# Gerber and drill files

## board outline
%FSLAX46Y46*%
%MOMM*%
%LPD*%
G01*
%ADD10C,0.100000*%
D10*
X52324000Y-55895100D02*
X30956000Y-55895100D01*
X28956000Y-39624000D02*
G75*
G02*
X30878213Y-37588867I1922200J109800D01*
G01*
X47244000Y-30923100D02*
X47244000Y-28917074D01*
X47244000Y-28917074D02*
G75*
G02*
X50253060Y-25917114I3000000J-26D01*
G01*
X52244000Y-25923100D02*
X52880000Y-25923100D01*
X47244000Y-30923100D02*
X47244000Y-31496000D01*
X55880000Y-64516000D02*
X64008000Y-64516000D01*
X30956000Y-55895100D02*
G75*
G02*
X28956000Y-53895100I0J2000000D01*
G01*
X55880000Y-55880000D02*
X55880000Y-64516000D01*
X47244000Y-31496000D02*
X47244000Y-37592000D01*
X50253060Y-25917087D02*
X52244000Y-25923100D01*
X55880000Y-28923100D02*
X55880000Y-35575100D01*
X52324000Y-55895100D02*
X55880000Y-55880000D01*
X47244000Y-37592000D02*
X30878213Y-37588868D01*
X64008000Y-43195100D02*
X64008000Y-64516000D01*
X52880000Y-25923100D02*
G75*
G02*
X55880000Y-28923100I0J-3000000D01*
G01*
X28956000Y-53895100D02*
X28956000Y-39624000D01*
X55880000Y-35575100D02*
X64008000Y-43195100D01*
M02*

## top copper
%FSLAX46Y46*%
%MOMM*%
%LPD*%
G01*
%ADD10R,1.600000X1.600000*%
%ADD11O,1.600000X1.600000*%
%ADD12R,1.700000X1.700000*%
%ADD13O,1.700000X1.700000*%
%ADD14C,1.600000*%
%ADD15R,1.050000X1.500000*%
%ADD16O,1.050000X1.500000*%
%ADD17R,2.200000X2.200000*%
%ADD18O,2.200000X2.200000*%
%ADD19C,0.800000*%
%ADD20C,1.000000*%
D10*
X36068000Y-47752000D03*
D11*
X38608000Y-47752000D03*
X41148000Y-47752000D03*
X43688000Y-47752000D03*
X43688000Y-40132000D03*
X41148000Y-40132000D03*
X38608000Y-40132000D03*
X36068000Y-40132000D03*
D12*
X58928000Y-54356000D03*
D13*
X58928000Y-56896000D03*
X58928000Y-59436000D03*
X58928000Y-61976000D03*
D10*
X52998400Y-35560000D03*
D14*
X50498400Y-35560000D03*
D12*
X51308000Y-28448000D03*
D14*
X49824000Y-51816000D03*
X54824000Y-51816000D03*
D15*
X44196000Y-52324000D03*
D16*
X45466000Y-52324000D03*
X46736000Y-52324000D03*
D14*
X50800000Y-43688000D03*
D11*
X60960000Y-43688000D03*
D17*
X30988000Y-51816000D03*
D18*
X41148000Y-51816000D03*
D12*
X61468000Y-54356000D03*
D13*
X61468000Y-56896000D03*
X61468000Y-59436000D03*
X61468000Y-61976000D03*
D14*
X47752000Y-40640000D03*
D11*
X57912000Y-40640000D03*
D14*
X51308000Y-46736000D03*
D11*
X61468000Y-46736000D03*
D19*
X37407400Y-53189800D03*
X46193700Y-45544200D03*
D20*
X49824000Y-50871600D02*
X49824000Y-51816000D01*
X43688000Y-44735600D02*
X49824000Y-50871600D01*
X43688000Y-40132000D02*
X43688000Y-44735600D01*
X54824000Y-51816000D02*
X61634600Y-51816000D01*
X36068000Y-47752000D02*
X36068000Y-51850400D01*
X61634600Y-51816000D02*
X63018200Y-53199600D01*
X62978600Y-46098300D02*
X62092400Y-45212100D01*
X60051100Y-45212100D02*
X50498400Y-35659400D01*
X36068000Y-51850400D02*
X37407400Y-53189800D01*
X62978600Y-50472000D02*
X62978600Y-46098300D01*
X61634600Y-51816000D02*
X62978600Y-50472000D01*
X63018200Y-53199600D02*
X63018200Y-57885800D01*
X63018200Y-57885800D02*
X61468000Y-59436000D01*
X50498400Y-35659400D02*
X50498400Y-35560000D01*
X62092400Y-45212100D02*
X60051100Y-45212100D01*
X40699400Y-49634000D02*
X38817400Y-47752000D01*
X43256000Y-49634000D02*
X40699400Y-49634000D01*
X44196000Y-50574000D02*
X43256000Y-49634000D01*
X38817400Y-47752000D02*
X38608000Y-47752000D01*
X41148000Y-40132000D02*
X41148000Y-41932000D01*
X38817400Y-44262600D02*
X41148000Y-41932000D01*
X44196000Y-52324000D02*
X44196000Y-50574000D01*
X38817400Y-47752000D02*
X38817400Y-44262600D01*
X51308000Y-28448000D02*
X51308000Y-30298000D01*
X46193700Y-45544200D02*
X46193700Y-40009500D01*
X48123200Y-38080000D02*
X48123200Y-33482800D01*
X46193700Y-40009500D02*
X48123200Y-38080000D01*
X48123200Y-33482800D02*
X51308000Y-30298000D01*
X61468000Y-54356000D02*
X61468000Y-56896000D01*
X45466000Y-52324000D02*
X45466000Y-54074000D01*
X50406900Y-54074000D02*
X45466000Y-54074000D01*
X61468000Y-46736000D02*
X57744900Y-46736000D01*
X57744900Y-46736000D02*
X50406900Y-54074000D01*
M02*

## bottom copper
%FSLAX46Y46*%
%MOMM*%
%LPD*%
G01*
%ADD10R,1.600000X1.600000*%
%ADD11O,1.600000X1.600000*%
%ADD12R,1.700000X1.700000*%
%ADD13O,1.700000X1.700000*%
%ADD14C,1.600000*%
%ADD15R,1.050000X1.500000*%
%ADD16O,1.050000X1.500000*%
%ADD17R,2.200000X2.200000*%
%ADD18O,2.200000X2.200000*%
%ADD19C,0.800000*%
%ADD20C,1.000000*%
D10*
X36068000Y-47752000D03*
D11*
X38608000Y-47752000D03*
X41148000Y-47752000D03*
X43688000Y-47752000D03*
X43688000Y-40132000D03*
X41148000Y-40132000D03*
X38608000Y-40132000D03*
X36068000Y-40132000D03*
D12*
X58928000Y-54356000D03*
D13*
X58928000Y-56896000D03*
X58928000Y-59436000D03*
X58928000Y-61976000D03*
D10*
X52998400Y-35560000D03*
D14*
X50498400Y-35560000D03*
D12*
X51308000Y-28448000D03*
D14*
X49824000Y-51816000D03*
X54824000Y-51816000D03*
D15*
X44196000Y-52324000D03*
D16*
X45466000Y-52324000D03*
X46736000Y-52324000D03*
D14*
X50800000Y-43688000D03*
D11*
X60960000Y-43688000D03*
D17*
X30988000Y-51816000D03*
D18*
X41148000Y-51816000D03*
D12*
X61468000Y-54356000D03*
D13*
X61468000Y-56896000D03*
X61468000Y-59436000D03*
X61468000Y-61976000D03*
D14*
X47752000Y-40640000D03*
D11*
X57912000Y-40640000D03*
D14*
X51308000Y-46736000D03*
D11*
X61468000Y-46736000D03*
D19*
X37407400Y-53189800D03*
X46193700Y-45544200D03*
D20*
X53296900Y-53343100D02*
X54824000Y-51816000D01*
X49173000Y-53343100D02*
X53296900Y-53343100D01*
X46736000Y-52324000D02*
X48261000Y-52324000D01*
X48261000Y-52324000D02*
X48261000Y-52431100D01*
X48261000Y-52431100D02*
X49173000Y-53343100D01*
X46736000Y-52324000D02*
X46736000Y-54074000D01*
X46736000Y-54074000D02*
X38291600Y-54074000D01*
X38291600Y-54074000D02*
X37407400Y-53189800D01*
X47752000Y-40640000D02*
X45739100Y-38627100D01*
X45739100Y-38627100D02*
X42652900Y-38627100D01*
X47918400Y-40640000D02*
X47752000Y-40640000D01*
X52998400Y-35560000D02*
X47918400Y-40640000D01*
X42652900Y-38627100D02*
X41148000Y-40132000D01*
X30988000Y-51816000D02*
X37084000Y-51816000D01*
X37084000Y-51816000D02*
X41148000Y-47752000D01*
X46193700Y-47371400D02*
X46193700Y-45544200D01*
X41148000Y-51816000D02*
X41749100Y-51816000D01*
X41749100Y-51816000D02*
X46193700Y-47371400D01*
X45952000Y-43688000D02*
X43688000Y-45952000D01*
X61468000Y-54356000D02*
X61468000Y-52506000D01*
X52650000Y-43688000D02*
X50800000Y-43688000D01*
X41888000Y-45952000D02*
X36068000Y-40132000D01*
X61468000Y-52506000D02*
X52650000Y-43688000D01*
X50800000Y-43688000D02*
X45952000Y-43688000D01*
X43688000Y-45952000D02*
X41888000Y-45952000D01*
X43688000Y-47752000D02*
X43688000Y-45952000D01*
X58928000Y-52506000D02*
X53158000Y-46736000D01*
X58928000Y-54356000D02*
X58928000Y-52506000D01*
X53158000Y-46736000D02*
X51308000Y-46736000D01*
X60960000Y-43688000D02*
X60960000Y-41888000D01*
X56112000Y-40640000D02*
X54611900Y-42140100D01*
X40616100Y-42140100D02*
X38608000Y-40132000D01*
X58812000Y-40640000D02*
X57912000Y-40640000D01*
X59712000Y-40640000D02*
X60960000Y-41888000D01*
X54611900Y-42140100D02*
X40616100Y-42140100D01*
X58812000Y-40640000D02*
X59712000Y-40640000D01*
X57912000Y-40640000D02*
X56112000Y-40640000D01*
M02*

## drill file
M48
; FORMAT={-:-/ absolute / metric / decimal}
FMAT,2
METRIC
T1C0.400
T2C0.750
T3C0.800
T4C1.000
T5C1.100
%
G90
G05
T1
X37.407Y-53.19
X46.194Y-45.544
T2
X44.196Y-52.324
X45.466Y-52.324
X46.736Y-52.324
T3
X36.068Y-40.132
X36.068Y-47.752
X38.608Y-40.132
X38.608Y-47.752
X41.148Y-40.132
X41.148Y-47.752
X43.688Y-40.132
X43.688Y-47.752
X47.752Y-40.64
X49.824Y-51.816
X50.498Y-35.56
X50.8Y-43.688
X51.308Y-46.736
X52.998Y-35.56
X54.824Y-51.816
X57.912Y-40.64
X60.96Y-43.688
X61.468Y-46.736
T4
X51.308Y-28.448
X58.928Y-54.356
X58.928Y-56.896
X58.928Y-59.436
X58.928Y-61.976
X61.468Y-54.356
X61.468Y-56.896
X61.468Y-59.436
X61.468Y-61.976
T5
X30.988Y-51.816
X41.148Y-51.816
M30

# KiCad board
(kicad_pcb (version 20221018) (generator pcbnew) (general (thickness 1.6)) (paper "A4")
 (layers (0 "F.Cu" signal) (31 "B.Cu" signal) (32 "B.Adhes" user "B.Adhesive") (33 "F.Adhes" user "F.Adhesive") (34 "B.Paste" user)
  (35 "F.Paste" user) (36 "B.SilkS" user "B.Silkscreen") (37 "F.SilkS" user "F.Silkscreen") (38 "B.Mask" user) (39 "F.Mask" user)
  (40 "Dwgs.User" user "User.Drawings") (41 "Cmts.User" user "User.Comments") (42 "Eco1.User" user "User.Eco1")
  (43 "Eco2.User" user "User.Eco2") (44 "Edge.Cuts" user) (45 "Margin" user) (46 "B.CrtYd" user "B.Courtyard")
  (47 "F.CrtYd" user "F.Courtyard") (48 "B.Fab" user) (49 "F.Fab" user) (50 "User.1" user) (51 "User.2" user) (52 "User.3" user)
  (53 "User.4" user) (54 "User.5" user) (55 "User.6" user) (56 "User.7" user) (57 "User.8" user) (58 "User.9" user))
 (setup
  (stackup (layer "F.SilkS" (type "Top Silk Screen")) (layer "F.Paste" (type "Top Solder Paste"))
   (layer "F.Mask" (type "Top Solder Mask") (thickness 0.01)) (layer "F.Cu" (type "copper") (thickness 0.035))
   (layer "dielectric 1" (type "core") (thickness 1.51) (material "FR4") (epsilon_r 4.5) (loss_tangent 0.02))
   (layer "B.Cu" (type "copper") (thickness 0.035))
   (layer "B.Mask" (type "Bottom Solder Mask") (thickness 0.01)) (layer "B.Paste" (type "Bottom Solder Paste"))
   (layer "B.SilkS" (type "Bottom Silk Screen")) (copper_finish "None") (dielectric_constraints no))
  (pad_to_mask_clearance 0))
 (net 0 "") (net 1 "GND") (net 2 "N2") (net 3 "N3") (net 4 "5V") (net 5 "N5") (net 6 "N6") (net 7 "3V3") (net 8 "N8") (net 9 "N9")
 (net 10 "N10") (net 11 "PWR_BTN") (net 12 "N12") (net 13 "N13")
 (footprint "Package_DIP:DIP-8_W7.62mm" (layer "F.Cu") (at 36.068 47.752 90)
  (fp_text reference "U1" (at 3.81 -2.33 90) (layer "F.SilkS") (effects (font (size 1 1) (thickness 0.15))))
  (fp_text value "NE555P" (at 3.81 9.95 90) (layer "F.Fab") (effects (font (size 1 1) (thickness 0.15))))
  (pad "1" thru_hole rect (at 0 0 90) (size 1.6 1.6) (drill 0.8) (layers "*.Cu" "*.Mask") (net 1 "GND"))
  (pad "2" thru_hole oval (at 0 2.54 90) (size 1.6 1.6) (drill 0.8) (layers "*.Cu" "*.Mask") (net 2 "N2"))
  (pad "3" thru_hole oval (at 0 5.08 90) (size 1.6 1.6) (drill 0.8) (layers "*.Cu" "*.Mask") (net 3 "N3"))
  (pad "4" thru_hole oval (at 0 7.62 90) (size 1.6 1.6) (drill 0.8) (layers "*.Cu" "*.Mask") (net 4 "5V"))
  (pad "5" thru_hole oval (at 7.62 7.62 90) (size 1.6 1.6) (drill 0.8) (layers "*.Cu" "*.Mask") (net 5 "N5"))
  (pad "6" thru_hole oval (at 7.62 5.08 90) (size 1.6 1.6) (drill 0.8) (layers "*.Cu" "*.Mask") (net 2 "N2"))
  (pad "7" thru_hole oval (at 7.62 2.54 90) (size 1.6 1.6) (drill 0.8) (layers "*.Cu" "*.Mask") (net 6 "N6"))
  (pad "8" thru_hole oval (at 7.62 0 90) (size 1.6 1.6) (drill 0.8) (layers "*.Cu" "*.Mask") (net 4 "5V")))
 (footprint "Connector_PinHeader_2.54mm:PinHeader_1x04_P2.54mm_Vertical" (layer "F.Cu") (at 58.928 54.356)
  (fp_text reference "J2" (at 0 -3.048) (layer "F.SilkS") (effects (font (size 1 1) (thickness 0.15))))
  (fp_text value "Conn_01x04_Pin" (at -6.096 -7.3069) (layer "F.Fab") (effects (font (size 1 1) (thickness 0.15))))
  (pad "1" thru_hole rect (at 0 0) (size 1.7 1.7) (drill 1) (layers "*.Cu" "*.Mask") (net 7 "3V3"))
  (pad "2" thru_hole oval (at 0 2.54) (size 1.7 1.7) (drill 1) (layers "*.Cu" "*.Mask") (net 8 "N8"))
  (pad "3" thru_hole oval (at 0 5.08) (size 1.7 1.7) (drill 1) (layers "*.Cu" "*.Mask") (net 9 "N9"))
  (pad "4" thru_hole oval (at 0 7.62) (size 1.7 1.7) (drill 1) (layers "*.Cu" "*.Mask") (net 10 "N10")))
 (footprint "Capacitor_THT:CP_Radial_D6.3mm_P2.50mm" (layer "F.Cu") (at 52.9984 35.56 180)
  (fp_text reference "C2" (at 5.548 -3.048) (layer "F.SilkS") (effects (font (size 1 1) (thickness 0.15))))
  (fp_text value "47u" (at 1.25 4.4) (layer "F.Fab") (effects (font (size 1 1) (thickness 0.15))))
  (pad "1" thru_hole rect (at 0 0 180) (size 1.6 1.6) (drill 0.8) (layers "*.Cu" "*.Mask") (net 2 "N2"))
  (pad "2" thru_hole circle (at 2.5 0 180) (size 1.6 1.6) (drill 0.8) (layers "*.Cu" "*.Mask") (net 1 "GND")))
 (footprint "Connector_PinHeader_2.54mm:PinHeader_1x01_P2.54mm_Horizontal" (layer "F.Cu") (at 51.308 28.448 90)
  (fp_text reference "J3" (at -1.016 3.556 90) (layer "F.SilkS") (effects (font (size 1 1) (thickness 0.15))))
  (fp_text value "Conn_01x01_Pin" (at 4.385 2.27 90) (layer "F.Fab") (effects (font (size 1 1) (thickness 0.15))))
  (pad "1" thru_hole rect (at 0 0 90) (size 1.7 1.7) (drill 1) (layers "*.Cu" "*.Mask") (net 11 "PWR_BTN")))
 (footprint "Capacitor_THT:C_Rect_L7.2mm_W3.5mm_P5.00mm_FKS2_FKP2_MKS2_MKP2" (layer "F.Cu") (at 49.824 51.816)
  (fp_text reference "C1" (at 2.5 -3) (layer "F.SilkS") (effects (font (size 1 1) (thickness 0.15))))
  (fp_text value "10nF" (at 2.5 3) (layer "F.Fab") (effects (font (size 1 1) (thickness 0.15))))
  (pad "1" thru_hole circle (at 0 0) (size 1.6 1.6) (drill 0.8) (layers "*.Cu" "*.Mask") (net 5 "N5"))
  (pad "2" thru_hole circle (at 5 0) (size 1.6 1.6) (drill 0.8) (layers "*.Cu" "*.Mask") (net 1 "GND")))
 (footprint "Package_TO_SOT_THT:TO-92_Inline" (layer "F.Cu") (at 44.196 52.324)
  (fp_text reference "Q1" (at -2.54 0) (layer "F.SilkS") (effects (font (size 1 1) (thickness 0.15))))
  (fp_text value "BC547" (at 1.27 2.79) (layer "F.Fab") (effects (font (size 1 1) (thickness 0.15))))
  (pad "1" thru_hole rect (at 0 0) (size 1.05 1.5) (drill 0.75) (layers "*.Cu" "*.Mask") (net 2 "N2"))
  (pad "2" thru_hole oval (at 1.27 0) (size 1.05 1.5) (drill 0.75) (layers "*.Cu" "*.Mask") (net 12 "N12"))
  (pad "3" thru_hole oval (at 2.54 0) (size 1.05 1.5) (drill 0.75) (layers "*.Cu" "*.Mask") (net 1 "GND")))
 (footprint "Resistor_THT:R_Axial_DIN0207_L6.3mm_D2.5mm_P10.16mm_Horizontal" (layer "F.Cu") (at 50.8 43.688)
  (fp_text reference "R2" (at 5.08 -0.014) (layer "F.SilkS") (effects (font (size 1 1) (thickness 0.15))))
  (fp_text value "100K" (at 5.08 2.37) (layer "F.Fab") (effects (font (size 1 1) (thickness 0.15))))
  (pad "1" thru_hole circle (at 0 0) (size 1.6 1.6) (drill 0.8) (layers "*.Cu" "*.Mask") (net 4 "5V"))
  (pad "2" thru_hole oval (at 10.16 0) (size 1.6 1.6) (drill 0.8) (layers "*.Cu" "*.Mask") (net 6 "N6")))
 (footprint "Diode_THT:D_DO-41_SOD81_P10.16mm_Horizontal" (layer "F.Cu") (at 30.988 51.816)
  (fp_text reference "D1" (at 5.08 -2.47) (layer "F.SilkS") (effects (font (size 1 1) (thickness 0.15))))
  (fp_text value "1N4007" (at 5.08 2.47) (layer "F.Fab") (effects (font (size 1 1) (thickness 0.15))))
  (pad "1" thru_hole rect (at 0 0) (size 2.2 2.2) (drill 1.1) (layers "*.Cu" "*.Mask") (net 3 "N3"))
  (pad "2" thru_hole oval (at 10.16 0) (size 2.2 2.2) (drill 1.1) (layers "*.Cu" "*.Mask") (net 11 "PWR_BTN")))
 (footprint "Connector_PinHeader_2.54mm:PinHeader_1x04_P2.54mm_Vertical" (layer "F.Cu") (at 61.468 54.356)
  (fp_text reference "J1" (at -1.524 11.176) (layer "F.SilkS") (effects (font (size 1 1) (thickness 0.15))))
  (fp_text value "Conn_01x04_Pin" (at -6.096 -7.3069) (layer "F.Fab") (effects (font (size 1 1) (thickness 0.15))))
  (pad "1" thru_hole rect (at 0 0) (size 1.7 1.7) (drill 1) (layers "*.Cu" "*.Mask") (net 4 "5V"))
  (pad "2" thru_hole oval (at 0 2.54) (size 1.7 1.7) (drill 1) (layers "*.Cu" "*.Mask") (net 4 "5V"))
  (pad "3" thru_hole oval (at 0 5.08) (size 1.7 1.7) (drill 1) (layers "*.Cu" "*.Mask") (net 1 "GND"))
  (pad "4" thru_hole oval (at 0 7.62) (size 1.7 1.7) (drill 1) (layers "*.Cu" "*.Mask") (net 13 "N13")))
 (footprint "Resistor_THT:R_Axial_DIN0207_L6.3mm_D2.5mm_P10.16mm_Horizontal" (layer "F.Cu") (at 47.752 40.64)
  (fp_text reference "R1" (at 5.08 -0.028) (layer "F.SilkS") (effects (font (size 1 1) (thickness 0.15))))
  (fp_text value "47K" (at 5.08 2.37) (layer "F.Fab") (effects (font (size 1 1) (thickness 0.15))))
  (pad "1" thru_hole circle (at 0 0) (size 1.6 1.6) (drill 0.8) (layers "*.Cu" "*.Mask") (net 2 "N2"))
  (pad "2" thru_hole oval (at 10.16 0) (size 1.6 1.6) (drill 0.8) (layers "*.Cu" "*.Mask") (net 6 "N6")))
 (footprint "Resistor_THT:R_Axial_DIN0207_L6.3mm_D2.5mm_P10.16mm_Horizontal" (layer "F.Cu") (at 51.308 46.736)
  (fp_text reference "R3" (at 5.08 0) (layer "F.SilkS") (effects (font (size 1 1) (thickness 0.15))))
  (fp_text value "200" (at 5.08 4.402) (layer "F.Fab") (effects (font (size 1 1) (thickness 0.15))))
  (pad "1" thru_hole circle (at 0 0) (size 1.6 1.6) (drill 0.8) (layers "*.Cu" "*.Mask") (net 7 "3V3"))
  (pad "2" thru_hole oval (at 10.16 0) (size 1.6 1.6) (drill 0.8) (layers "*.Cu" "*.Mask") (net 12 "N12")))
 (gr_line (start 52.324 55.8951) (end 30.956 55.8951) (stroke (width 0.1) (type default)) (layer "Edge.Cuts"))
 (gr_arc (start 28.956 39.624) (mid 29.478511 38.192174) (end 30.878213 37.588868) (stroke (width 0.1) (type default)) (layer "Edge.Cuts"))
 (gr_line (start 47.244 30.9231) (end 47.244 28.917074) (stroke (width 0.1) (type default)) (layer "Edge.Cuts"))
 (gr_arc (start 47.244 28.917074) (mid 48.125894 26.79257) (end 50.25306 25.917087) (stroke (width 0.1) (type default)) (layer "Edge.Cuts"))
 (gr_line (start 52.244 25.9231) (end 52.88 25.9231) (stroke (width 0.1) (type default)) (layer "Edge.Cuts"))
 (gr_line (start 47.244 30.9231) (end 47.244 31.496) (stroke (width 0.1) (type default)) (layer "Edge.Cuts"))
 (gr_line (start 55.88 64.516) (end 64.008 64.516) (stroke (width 0.1) (type default)) (layer "Edge.Cuts"))
 (gr_arc (start 30.956 55.8951) (mid 29.541786 55.309314) (end 28.956 53.8951) (stroke (width 0.1) (type default)) (layer "Edge.Cuts"))
 (gr_line (start 55.88 55.88) (end 55.88 64.516) (stroke (width 0.1) (type default)) (layer "Edge.Cuts"))
 (gr_line (start 47.244 31.496) (end 47.244 37.592) (stroke (width 0.1) (type default)) (layer "Edge.Cuts"))
 (gr_line (start 50.25306 25.917087) (end 52.244 25.9231) (stroke (width 0.1) (type default)) (layer "Edge.Cuts"))
 (gr_line (start 55.88 28.9231) (end 55.88 35.5751) (stroke (width 0.1) (type default)) (layer "Edge.Cuts"))
 (gr_line (start 52.324 55.8951) (end 55.88 55.88) (stroke (width 0.1) (type default)) (layer "Edge.Cuts"))
 (gr_line (start 47.244 37.592) (end 30.878213 37.588868) (stroke (width 0.1) (type default)) (layer "Edge.Cuts"))
 (gr_line (start 64.008 43.1951) (end 64.008 64.516) (stroke (width 0.1) (type default)) (layer "Edge.Cuts"))
 (gr_arc (start 52.88 25.9231) (mid 55.00132 26.80178) (end 55.88 28.9231) (stroke (width 0.1) (type default)) (layer "Edge.Cuts"))
 (gr_line (start 28.956 53.8951) (end 28.956 39.624) (stroke (width 0.1) (type default)) (layer "Edge.Cuts"))
 (gr_line (start 55.88 35.5751) (end 64.008 43.1951) (stroke (width 0.1) (type default)) (layer "Edge.Cuts"))
 (segment (start 49.824 50.8716) (end 49.824 51.816) (width 1) (layer "F.Cu") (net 5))
 (segment (start 43.688 44.7356) (end 49.824 50.8716) (width 1) (layer "F.Cu") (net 5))
 (segment (start 43.688 40.132) (end 43.688 44.7356) (width 1) (layer "F.Cu") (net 5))
 (segment (start 54.824 51.816) (end 61.6346 51.816) (width 1) (layer "F.Cu") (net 1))
 (segment (start 36.068 47.752) (end 36.068 51.8504) (width 1) (layer "F.Cu") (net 1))
 (segment (start 61.6346 51.816) (end 63.0182 53.1996) (width 1) (layer "F.Cu") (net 1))
 (segment (start 62.9786 46.0983) (end 62.0924 45.2121) (width 1) (layer "F.Cu") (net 1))
 (segment (start 60.0511 45.2121) (end 50.4984 35.6594) (width 1) (layer "F.Cu") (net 1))
 (segment (start 36.068 51.8504) (end 37.4074 53.1898) (width 1) (layer "F.Cu") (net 1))
 (segment (start 62.9786 50.472) (end 62.9786 46.0983) (width 1) (layer "F.Cu") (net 1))
 (segment (start 61.6346 51.816) (end 62.9786 50.472) (width 1) (layer "F.Cu") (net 1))
 (segment (start 63.0182 53.1996) (end 63.0182 57.8858) (width 1) (layer "F.Cu") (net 1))
 (segment (start 63.0182 57.8858) (end 61.468 59.436) (width 1) (layer "F.Cu") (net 1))
 (segment (start 50.4984 35.6594) (end 50.4984 35.56) (width 1) (layer "F.Cu") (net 1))
 (segment (start 62.0924 45.2121) (end 60.0511 45.2121) (width 1) (layer "F.Cu") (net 1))
 (via (at 37.4074 53.1898) (size 0.8) (drill 0.4) (layers "F.Cu" "B.Cu") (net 1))
 (segment (start 53.2969 53.3431) (end 54.824 51.816) (width 1) (layer "B.Cu") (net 1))
 (segment (start 49.173 53.3431) (end 53.2969 53.3431) (width 1) (layer "B.Cu") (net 1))
 (segment (start 46.736 52.324) (end 48.261 52.324) (width 1) (layer "B.Cu") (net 1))
 (segment (start 48.261 52.324) (end 48.261 52.4311) (width 1) (layer "B.Cu") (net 1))
 (segment (start 48.261 52.4311) (end 49.173 53.3431) (width 1) (layer "B.Cu") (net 1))
 (segment (start 46.736 52.324) (end 46.736 54.074) (width 1) (layer "B.Cu") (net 1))
 (segment (start 46.736 54.074) (end 38.2916 54.074) (width 1) (layer "B.Cu") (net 1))
 (segment (start 38.2916 54.074) (end 37.4074 53.1898) (width 1) (layer "B.Cu") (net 1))
 (segment (start 40.6994 49.634) (end 38.8174 47.752) (width 1) (layer "F.Cu") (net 2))
 (segment (start 43.256 49.634) (end 40.6994 49.634) (width 1) (layer "F.Cu") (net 2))
 (segment (start 44.196 50.574) (end 43.256 49.634) (width 1) (layer "F.Cu") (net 2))
 (segment (start 38.8174 47.752) (end 38.608 47.752) (width 1) (layer "F.Cu") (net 2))
 (segment (start 41.148 40.132) (end 41.148 41.932) (width 1) (layer "F.Cu") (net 2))
 (segment (start 38.8174 44.2626) (end 41.148 41.932) (width 1) (layer "F.Cu") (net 2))
 (segment (start 44.196 52.324) (end 44.196 50.574) (width 1) (layer "F.Cu") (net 2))
 (segment (start 38.8174 47.752) (end 38.8174 44.2626) (width 1) (layer "F.Cu") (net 2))
 (segment (start 47.752 40.64) (end 45.7391 38.6271) (width 1) (layer "B.Cu") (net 2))
 (segment (start 45.7391 38.6271) (end 42.6529 38.6271) (width 1) (layer "B.Cu") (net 2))
 (segment (start 47.9184 40.64) (end 47.752 40.64) (width 1) (layer "B.Cu") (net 2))
 (segment (start 52.9984 35.56) (end 47.9184 40.64) (width 1) (layer "B.Cu") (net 2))
 (segment (start 42.6529 38.6271) (end 41.148 40.132) (width 1) (layer "B.Cu") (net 2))
 (segment (start 30.988 51.816) (end 37.084 51.816) (width 1) (layer "B.Cu") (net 3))
 (segment (start 37.084 51.816) (end 41.148 47.752) (width 1) (layer "B.Cu") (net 3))
 (segment (start 51.308 28.448) (end 51.308 30.298) (width 1) (layer "F.Cu") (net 11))
 (segment (start 46.1937 45.5442) (end 46.1937 40.0095) (width 1) (layer "F.Cu") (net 11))
 (segment (start 48.1232 38.08) (end 48.1232 33.4828) (width 1) (layer "F.Cu") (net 11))
 (segment (start 46.1937 40.0095) (end 48.1232 38.08) (width 1) (layer "F.Cu") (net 11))
 (segment (start 48.1232 33.4828) (end 51.308 30.298) (width 1) (layer "F.Cu") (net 11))
 (via (at 46.1937 45.5442) (size 0.8) (drill 0.4) (layers "F.Cu" "B.Cu") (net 11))
 (segment (start 46.1937 47.3714) (end 46.1937 45.5442) (width 1) (layer "B.Cu") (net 11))
 (segment (start 41.148 51.816) (end 41.7491 51.816) (width 1) (layer "B.Cu") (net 11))
 (segment (start 41.7491 51.816) (end 46.1937 47.3714) (width 1) (layer "B.Cu") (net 11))
 (segment (start 61.468 54.356) (end 61.468 56.896) (width 1) (layer "F.Cu") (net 4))
 (segment (start 45.952 43.688) (end 43.688 45.952) (width 1) (layer "B.Cu") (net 4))
 (segment (start 61.468 54.356) (end 61.468 52.506) (width 1) (layer "B.Cu") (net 4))
 (segment (start 52.65 43.688) (end 50.8 43.688) (width 1) (layer "B.Cu") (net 4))
 (segment (start 41.888 45.952) (end 36.068 40.132) (width 1) (layer "B.Cu") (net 4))
 (segment (start 61.468 52.506) (end 52.65 43.688) (width 1) (layer "B.Cu") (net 4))
 (segment (start 50.8 43.688) (end 45.952 43.688) (width 1) (layer "B.Cu") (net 4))
 (segment (start 43.688 45.952) (end 41.888 45.952) (width 1) (layer "B.Cu") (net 4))
 (segment (start 43.688 47.752) (end 43.688 45.952) (width 1) (layer "B.Cu") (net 4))
 (segment (start 58.928 52.506) (end 53.158 46.736) (width 1) (layer "B.Cu") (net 7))
 (segment (start 58.928 54.356) (end 58.928 52.506) (width 1) (layer "B.Cu") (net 7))
 (segment (start 53.158 46.736) (end 51.308 46.736) (width 1) (layer "B.Cu") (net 7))
 (segment (start 45.466 52.324) (end 45.466 54.074) (width 1) (layer "F.Cu") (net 12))
 (segment (start 50.4069 54.074) (end 45.466 54.074) (width 1) (layer "F.Cu") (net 12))
 (segment (start 61.468 46.736) (end 57.7449 46.736) (width 1) (layer "F.Cu") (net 12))
 (segment (start 57.7449 46.736) (end 50.4069 54.074) (width 1) (layer "F.Cu") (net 12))
 (segment (start 60.96 43.688) (end 60.96 41.888) (width 1) (layer "B.Cu") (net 6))
 (segment (start 56.112 40.64) (end 54.6119 42.1401) (width 1) (layer "B.Cu") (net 6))
 (segment (start 40.6161 42.1401) (end 38.608 40.132) (width 1) (layer "B.Cu") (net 6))
 (segment (start 58.812 40.64) (end 57.912 40.64) (width 1) (layer "B.Cu") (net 6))
 (segment (start 59.712 40.64) (end 60.96 41.888) (width 1) (layer "B.Cu") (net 6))
 (segment (start 54.6119 42.1401) (end 40.6161 42.1401) (width 1) (layer "B.Cu") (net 6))
 (segment (start 58.812 40.64) (end 59.712 40.64) (width 1) (layer "B.Cu") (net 6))
 (segment (start 57.912 40.64) (end 56.112 40.64) (width 1) (layer "B.Cu") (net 6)))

